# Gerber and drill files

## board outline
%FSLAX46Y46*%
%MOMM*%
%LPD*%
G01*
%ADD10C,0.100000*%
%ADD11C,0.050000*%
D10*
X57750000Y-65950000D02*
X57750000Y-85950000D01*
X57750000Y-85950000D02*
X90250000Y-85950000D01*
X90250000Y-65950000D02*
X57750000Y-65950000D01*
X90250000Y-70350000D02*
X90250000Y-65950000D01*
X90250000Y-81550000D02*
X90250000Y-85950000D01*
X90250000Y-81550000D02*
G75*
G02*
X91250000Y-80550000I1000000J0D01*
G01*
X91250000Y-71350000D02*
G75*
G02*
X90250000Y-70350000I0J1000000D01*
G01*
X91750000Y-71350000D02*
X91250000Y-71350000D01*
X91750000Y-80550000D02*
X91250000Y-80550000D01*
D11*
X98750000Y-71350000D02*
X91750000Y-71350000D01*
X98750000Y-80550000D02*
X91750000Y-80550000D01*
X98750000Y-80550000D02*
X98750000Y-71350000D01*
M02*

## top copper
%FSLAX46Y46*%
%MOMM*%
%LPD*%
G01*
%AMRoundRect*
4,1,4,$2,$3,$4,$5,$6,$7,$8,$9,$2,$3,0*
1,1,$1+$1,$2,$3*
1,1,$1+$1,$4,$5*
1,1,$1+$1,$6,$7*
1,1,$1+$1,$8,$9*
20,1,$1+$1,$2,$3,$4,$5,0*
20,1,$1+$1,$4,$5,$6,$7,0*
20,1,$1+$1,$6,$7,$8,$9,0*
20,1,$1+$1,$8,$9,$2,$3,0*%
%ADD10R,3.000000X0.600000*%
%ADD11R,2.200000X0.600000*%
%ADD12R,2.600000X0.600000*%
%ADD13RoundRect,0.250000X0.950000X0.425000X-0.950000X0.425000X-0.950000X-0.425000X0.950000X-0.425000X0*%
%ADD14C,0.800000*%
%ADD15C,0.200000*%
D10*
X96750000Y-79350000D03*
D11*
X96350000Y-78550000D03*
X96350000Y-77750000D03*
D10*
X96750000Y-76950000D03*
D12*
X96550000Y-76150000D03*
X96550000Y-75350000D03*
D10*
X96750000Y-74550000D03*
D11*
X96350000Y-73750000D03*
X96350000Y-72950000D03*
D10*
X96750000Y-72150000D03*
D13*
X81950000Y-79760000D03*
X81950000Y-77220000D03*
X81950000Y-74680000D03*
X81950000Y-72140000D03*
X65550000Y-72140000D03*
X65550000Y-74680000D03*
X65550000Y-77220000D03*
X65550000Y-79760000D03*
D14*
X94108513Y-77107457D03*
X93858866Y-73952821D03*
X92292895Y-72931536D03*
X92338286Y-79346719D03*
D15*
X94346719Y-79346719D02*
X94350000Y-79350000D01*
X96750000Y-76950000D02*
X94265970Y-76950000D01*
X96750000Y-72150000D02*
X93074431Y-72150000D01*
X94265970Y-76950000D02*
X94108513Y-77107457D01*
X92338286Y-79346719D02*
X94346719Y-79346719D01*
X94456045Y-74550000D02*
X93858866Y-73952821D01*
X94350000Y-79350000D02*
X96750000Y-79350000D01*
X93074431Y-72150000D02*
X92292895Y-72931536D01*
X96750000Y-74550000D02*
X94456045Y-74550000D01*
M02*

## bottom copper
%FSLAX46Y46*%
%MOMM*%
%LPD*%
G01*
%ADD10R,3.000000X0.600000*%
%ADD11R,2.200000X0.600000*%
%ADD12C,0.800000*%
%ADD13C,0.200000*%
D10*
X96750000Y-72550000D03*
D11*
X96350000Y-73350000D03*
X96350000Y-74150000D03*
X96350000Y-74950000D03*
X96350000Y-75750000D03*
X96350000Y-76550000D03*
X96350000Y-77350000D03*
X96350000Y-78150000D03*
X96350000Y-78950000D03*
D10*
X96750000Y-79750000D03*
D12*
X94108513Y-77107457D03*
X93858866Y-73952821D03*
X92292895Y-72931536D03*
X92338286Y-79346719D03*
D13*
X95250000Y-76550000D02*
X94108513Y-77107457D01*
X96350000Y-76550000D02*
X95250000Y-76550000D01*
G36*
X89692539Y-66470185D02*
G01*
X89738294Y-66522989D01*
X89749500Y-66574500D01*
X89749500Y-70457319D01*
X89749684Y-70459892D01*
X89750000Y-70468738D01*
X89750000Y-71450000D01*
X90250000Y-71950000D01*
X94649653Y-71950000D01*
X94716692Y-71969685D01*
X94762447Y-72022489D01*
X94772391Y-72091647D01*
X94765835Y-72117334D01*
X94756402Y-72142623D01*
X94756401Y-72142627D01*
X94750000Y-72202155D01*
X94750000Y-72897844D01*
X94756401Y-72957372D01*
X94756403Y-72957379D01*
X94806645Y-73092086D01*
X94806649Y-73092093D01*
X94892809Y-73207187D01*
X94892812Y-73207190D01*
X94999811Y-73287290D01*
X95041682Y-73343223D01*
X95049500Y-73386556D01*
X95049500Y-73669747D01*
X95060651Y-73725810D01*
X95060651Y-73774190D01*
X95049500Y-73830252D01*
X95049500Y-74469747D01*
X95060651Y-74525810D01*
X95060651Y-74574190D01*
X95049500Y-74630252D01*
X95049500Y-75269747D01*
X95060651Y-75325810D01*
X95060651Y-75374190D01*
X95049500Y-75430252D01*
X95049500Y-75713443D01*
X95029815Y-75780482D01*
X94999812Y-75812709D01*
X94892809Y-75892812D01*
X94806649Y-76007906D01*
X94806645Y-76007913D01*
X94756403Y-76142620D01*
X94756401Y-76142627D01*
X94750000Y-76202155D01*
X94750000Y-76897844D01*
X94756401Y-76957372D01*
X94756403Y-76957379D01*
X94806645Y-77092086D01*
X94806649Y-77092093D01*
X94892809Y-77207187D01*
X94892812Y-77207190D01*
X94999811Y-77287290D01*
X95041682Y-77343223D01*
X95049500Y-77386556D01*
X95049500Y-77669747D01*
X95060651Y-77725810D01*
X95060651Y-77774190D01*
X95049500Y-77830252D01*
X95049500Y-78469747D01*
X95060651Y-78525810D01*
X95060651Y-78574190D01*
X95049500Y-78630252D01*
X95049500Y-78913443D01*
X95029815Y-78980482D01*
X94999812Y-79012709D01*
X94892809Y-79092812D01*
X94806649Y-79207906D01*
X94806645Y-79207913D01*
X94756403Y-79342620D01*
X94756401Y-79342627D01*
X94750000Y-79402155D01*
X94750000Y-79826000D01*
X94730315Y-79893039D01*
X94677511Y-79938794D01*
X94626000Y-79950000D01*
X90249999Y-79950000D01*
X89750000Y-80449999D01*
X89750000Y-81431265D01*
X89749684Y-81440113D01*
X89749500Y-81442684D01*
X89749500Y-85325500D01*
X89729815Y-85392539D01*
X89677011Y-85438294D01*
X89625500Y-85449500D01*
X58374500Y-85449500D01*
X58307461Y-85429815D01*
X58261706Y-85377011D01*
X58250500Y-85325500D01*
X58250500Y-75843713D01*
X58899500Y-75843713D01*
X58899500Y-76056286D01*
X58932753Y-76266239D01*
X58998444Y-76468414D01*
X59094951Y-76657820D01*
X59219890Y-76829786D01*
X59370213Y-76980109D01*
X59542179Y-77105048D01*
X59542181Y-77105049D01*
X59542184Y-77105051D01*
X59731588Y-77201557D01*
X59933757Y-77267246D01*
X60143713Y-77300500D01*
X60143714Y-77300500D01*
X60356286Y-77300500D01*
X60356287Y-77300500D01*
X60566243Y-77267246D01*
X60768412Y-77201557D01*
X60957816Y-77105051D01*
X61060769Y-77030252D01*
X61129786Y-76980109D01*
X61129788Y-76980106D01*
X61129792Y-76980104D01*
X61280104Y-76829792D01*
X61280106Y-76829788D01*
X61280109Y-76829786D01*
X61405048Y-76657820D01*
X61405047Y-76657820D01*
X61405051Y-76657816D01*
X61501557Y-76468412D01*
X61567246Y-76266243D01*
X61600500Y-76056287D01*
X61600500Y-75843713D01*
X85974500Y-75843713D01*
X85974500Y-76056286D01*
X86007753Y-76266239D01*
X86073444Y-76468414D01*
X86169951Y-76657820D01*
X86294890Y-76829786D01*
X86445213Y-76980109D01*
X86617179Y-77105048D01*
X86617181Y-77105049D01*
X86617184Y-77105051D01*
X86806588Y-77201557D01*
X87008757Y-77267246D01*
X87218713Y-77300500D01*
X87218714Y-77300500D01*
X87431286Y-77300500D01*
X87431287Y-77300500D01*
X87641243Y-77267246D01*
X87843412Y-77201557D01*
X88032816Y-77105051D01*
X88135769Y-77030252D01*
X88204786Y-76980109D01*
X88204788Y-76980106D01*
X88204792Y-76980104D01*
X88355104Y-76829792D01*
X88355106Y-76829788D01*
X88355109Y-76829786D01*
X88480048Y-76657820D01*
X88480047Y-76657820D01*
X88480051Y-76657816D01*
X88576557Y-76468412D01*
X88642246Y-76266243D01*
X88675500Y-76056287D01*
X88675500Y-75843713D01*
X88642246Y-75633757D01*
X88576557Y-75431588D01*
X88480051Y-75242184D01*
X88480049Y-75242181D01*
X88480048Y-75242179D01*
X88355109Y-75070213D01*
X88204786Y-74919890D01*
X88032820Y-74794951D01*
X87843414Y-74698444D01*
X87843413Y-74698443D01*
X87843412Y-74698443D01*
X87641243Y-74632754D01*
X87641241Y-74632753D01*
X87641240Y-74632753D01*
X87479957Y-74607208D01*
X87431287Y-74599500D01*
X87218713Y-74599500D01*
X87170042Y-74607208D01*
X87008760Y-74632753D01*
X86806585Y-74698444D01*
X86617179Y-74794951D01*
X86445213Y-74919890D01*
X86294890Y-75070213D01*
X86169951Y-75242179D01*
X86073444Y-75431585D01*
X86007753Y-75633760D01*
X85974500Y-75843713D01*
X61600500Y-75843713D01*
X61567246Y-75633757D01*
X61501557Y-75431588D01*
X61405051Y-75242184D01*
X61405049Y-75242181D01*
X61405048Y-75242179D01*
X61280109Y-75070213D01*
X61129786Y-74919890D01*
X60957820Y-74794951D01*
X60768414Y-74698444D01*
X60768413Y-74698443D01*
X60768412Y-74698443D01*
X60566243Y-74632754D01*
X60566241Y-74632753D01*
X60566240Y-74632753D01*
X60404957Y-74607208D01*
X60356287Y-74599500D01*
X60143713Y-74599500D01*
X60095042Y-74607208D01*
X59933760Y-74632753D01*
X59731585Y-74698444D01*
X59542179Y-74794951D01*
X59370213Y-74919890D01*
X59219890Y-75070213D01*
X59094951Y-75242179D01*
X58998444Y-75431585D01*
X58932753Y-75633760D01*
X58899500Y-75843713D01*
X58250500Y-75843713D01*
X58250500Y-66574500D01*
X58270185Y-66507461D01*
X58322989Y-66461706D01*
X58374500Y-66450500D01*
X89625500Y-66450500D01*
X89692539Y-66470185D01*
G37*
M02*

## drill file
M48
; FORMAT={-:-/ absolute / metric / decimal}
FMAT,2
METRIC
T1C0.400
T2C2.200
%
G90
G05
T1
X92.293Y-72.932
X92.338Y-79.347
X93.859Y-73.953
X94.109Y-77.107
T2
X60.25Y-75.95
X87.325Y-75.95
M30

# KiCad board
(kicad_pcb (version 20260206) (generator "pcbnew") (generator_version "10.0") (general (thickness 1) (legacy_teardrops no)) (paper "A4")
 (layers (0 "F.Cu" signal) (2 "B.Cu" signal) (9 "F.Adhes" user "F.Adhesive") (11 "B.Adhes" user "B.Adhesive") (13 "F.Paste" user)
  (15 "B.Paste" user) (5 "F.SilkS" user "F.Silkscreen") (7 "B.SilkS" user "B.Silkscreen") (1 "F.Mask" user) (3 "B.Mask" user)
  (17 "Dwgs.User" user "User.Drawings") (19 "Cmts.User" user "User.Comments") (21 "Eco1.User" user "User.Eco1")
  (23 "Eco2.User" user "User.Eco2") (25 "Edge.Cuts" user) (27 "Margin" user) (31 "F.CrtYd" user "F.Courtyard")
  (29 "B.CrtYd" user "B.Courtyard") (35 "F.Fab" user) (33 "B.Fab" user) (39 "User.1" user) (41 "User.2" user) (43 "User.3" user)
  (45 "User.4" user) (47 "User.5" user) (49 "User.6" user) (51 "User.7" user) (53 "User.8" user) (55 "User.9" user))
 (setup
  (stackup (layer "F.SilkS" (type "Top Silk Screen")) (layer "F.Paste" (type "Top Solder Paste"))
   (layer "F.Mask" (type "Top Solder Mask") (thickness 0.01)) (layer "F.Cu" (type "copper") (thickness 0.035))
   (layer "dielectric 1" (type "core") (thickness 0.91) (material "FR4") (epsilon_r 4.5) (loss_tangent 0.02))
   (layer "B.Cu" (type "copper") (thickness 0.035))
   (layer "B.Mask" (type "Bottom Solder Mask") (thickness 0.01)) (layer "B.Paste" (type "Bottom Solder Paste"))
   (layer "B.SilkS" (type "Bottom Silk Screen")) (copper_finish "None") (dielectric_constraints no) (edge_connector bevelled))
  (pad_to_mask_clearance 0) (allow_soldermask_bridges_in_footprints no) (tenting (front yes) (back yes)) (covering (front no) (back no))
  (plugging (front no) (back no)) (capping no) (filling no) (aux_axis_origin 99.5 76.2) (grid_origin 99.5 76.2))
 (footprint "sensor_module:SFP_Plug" (layer "F.Cu") (at 95.25 75.95)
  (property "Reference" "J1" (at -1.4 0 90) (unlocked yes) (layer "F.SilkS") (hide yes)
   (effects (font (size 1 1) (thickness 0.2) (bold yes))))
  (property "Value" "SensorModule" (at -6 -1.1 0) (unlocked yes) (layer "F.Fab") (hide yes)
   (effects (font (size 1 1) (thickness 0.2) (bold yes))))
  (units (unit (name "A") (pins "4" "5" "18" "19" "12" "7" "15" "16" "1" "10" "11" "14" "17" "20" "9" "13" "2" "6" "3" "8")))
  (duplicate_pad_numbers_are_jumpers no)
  (fp_line (start 3.5 -4.6) (end -3.5 -4.6) (stroke (width 0.05) (type solid)) (layer "Edge.Cuts"))
  (fp_line (start 3.5 4.6) (end -3.5 4.6) (stroke (width 0.05) (type solid)) (layer "Edge.Cuts"))
  (fp_line (start 3.5 4.6) (end 3.5 -4.6) (stroke (width 0.05) (type default)) (layer "Edge.Cuts"))
  (pad "1" smd rect (at 1.5 -3.4) (size 3 0.6) (layers "B.Cu" "B.Mask") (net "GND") (thermal_bridge_angle 45))
  (pad "2" smd rect (at 1.1 -2.6) (size 2.2 0.6) (layers "B.Cu" "B.Mask") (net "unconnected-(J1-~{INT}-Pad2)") (thermal_bridge_angle 45))
  (pad "3" smd rect (at 1.1 -1.8) (size 2.2 0.6) (layers "B.Cu" "B.Mask") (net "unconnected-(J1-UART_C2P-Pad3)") (thermal_bridge_angle 45))
  (pad "4" smd rect (at 1.1 -1) (size 2.2 0.6) (layers "B.Cu" "B.Mask") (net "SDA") (thermal_bridge_angle 45))
  (pad "5" smd rect (at 1.1 -0.2) (size 2.2 0.6) (layers "B.Cu" "B.Mask") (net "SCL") (thermal_bridge_angle 45))
  (pad "6" smd rect (at 1.1 0.6) (size 2.2 0.6) (layers "B.Cu" "B.Mask") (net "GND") (thermal_bridge_angle 45))
  (pad "7" smd rect (at 1.1 1.4) (size 2.2 0.6) (layers "B.Cu" "B.Mask") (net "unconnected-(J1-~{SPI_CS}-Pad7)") (thermal_bridge_angle 45))
  (pad "8" smd rect (at 1.1 2.2) (size 2.2 0.6) (layers "B.Cu" "B.Mask") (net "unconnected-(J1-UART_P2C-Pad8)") (thermal_bridge_angle 45))
  (pad "9" smd rect (at 1.1 3) (size 2.2 0.6) (layers "B.Cu" "B.Mask") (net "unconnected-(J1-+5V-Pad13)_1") (thermal_bridge_angle 45))
  (pad "10" smd rect (at 1.5 3.8) (size 3 0.6) (layers "B.Cu" "B.Mask") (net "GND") (thermal_bridge_angle 45))
  (pad "11" smd rect (at 1.5 3.4) (size 3 0.6) (layers "F.Cu" "F.Mask") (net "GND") (thermal_bridge_angle 45))
  (pad "12" smd rect (at 1.1 2.6) (size 2.2 0.6) (layers "F.Cu" "F.Mask") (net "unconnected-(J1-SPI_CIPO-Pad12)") (thermal_bridge_angle 45))
  (pad "13" smd rect (at 1.1 1.8) (size 2.2 0.6) (layers "F.Cu" "F.Mask") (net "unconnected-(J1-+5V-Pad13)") (thermal_bridge_angle 45))
  (pad "14" smd rect (at 1.5 1) (size 3 0.6) (layers "F.Cu" "F.Mask") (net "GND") (thermal_bridge_angle 45))
  (pad "15" smd rect (at 1.3 0.2) (size 2.6 0.6) (layers "F.Cu" "F.Mask") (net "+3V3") (thermal_bridge_angle 45))
  (pad "16" smd rect (at 1.3 -0.6) (size 2.6 0.6) (layers "F.Cu" "F.Mask") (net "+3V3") (thermal_bridge_angle 45))
  (pad "17" smd rect (at 1.5 -1.4) (size 3 0.6) (layers "F.Cu" "F.Mask") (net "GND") (thermal_bridge_angle 45))
  (pad "18" smd rect (at 1.1 -2.2) (size 2.2 0.6) (layers "F.Cu" "F.Mask") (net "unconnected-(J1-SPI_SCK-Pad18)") (thermal_bridge_angle 45))
  (pad "19" smd rect (at 1.1 -3) (size 2.2 0.6) (layers "F.Cu" "F.Mask") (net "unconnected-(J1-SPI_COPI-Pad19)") (thermal_bridge_angle 45))
  (pad "20" smd rect (at 1.5 -3.8) (size 3 0.6) (layers "F.Cu" "F.Mask") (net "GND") (thermal_bridge_angle 45)))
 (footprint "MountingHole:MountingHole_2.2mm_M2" (layer "F.Cu") (at 60.25 75.95 180)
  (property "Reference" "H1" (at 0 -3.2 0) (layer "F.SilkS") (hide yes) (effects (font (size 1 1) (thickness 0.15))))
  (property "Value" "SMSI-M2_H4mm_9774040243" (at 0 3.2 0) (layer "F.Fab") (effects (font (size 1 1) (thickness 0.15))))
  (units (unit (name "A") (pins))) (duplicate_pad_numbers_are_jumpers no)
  (pad "" np_thru_hole circle (at 0 0 180) (size 2.2 2.2) (drill 2.2) (layers "*.Cu" "*.Mask")))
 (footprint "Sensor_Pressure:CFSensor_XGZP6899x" (layer "F.Cu") (at 73.75 75.95 180)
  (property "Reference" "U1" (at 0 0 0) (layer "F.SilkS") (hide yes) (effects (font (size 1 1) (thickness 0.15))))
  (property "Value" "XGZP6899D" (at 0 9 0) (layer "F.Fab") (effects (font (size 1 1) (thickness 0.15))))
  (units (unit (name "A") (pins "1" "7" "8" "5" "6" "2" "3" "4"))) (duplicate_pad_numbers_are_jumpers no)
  (pad "1" smd roundrect (at -8.2 -3.81 180) (size 2.4 1.35) (layers "F.Cu" "F.Mask" "F.Paste") (roundrect_rratio 0.185185)
   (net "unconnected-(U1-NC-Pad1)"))
  (pad "2" smd roundrect (at -8.2 -1.27 180) (size 2.4 1.35) (layers "F.Cu" "F.Mask" "F.Paste") (roundrect_rratio 0.185185) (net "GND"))
  (pad "3" smd roundrect (at -8.2 1.27 180) (size 2.4 1.35) (layers "F.Cu" "F.Mask" "F.Paste") (roundrect_rratio 0.185185) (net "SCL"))
  (pad "4" smd roundrect (at -8.2 3.81 180) (size 2.4 1.35) (layers "F.Cu" "F.Mask" "F.Paste") (roundrect_rratio 0.185185) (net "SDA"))
  (pad "5" smd roundrect (at 8.2 3.81 180) (size 2.4 1.35) (layers "F.Cu" "F.Mask" "F.Paste") (roundrect_rratio 0.185185)
   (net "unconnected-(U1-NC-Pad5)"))
  (pad "6" smd roundrect (at 8.2 1.27 180) (size 2.4 1.35) (layers "F.Cu" "F.Mask" "F.Paste") (roundrect_rratio 0.185185) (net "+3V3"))
  (pad "7" smd roundrect (at 8.2 -1.27 180) (size 2.4 1.35) (layers "F.Cu" "F.Mask" "F.Paste") (roundrect_rratio 0.185185)
   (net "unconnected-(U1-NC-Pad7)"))
  (pad "8" smd roundrect (at 8.2 -3.81 180) (size 2.4 1.35) (layers "F.Cu" "F.Mask" "F.Paste") (roundrect_rratio 0.185185)
   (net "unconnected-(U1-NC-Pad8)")))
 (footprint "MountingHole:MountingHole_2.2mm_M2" (layer "F.Cu") (at 87.325 75.95 180)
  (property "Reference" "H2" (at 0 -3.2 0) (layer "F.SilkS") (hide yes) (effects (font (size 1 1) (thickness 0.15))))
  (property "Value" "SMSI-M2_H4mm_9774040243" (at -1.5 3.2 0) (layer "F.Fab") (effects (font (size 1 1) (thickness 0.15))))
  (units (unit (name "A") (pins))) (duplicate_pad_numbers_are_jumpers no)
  (pad "" np_thru_hole circle (at 0 0 180) (size 2.2 2.2) (drill 2.2) (layers "*.Cu" "*.Mask")))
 (gr_line (start 57.75 65.95) (end 57.75 85.95) (stroke (width 0.1) (type default)) (layer "Edge.Cuts"))
 (gr_line (start 57.75 85.95) (end 90.25 85.95) (stroke (width 0.1) (type default)) (layer "Edge.Cuts"))
 (gr_line (start 90.25 65.95) (end 57.75 65.95) (stroke (width 0.1) (type default)) (layer "Edge.Cuts"))
 (gr_line (start 90.25 70.35) (end 90.25 65.95) (stroke (width 0.1) (type default)) (layer "Edge.Cuts"))
 (gr_line (start 90.25 81.55) (end 90.25 85.95) (stroke (width 0.1) (type default)) (layer "Edge.Cuts"))
 (gr_arc (start 90.25 81.55) (mid 90.542893 80.842893) (end 91.25 80.55) (stroke (width 0.1) (type default)) (layer "Edge.Cuts"))
 (gr_arc (start 91.25 71.35) (mid 90.542893 71.057107) (end 90.25 70.35) (stroke (width 0.1) (type default)) (layer "Edge.Cuts"))
 (gr_line (start 91.75 71.35) (end 91.25 71.35) (stroke (width 0.1) (type default)) (layer "Edge.Cuts"))
 (gr_line (start 91.75 80.55) (end 91.25 80.55) (stroke (width 0.1) (type default)) (layer "Edge.Cuts"))
 (segment (start 94.346719 79.346719) (end 94.35 79.35) (width 0.2) (layer "F.Cu") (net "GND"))
 (segment (start 96.75 76.95) (end 94.26597 76.95) (width 0.2) (layer "F.Cu") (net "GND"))
 (segment (start 96.75 72.15) (end 93.074431 72.15) (width 0.2) (layer "F.Cu") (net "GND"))
 (segment (start 94.26597 76.95) (end 94.108513 77.107457) (width 0.2) (layer "F.Cu") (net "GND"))
 (segment (start 92.338286 79.346719) (end 94.346719 79.346719) (width 0.2) (layer "F.Cu") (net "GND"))
 (segment (start 94.456045 74.55) (end 93.858866 73.952821) (width 0.2) (layer "F.Cu") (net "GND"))
 (segment (start 94.35 79.35) (end 96.75 79.35) (width 0.2) (layer "F.Cu") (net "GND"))
 (segment (start 93.074431 72.15) (end 92.292895 72.931536) (width 0.2) (layer "F.Cu") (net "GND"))
 (segment (start 96.75 74.55) (end 94.456045 74.55) (width 0.2) (layer "F.Cu") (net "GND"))
 (via (at 94.108513 77.107457) (size 0.8) (drill 0.4) (layers "F.Cu" "B.Cu") (capping no) (covering (front no) (back no))
  (plugging (front no) (back no)) (filling no) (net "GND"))
 (via (at 93.858866 73.952821) (size 0.8) (drill 0.4) (layers "F.Cu" "B.Cu") (capping no) (covering (front no) (back no))
  (plugging (front no) (back no)) (filling no) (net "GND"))
 (via (at 92.292895 72.931536) (size 0.8) (drill 0.4) (layers "F.Cu" "B.Cu") (capping no) (covering (front no) (back no))
  (plugging (front no) (back no)) (filling no) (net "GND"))
 (via (at 92.338286 79.346719) (size 0.8) (drill 0.4) (layers "F.Cu" "B.Cu") (capping no) (covering (front no) (back no))
  (plugging (front no) (back no)) (filling no) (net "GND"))
 (segment (start 95.25 76.55) (end 94.108513 77.107457) (width 0.2) (layer "B.Cu") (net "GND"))
 (segment (start 96.35 76.55) (end 95.25 76.55) (width 0.2) (layer "B.Cu") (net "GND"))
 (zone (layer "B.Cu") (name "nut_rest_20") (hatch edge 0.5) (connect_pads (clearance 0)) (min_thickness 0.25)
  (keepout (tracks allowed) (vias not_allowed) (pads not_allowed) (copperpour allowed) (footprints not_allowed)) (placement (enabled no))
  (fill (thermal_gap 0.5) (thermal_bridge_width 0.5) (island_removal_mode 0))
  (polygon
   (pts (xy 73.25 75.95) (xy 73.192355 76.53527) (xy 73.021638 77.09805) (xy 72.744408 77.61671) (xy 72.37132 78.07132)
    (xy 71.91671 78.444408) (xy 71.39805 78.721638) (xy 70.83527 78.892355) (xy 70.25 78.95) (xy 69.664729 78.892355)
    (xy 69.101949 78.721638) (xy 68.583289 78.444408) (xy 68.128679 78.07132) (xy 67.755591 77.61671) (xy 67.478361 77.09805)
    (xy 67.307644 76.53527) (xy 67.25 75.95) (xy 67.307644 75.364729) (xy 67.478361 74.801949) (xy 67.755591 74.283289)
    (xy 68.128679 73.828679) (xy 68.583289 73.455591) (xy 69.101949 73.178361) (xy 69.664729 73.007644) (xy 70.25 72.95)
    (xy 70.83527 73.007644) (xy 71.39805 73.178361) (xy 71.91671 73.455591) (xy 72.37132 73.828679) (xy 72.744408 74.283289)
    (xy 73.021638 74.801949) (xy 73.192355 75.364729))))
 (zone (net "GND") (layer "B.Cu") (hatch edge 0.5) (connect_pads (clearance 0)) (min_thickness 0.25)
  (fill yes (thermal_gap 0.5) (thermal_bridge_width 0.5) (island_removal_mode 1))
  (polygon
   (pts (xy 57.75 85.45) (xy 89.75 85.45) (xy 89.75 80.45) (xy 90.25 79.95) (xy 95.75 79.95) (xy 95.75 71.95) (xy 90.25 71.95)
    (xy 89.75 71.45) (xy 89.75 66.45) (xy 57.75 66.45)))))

